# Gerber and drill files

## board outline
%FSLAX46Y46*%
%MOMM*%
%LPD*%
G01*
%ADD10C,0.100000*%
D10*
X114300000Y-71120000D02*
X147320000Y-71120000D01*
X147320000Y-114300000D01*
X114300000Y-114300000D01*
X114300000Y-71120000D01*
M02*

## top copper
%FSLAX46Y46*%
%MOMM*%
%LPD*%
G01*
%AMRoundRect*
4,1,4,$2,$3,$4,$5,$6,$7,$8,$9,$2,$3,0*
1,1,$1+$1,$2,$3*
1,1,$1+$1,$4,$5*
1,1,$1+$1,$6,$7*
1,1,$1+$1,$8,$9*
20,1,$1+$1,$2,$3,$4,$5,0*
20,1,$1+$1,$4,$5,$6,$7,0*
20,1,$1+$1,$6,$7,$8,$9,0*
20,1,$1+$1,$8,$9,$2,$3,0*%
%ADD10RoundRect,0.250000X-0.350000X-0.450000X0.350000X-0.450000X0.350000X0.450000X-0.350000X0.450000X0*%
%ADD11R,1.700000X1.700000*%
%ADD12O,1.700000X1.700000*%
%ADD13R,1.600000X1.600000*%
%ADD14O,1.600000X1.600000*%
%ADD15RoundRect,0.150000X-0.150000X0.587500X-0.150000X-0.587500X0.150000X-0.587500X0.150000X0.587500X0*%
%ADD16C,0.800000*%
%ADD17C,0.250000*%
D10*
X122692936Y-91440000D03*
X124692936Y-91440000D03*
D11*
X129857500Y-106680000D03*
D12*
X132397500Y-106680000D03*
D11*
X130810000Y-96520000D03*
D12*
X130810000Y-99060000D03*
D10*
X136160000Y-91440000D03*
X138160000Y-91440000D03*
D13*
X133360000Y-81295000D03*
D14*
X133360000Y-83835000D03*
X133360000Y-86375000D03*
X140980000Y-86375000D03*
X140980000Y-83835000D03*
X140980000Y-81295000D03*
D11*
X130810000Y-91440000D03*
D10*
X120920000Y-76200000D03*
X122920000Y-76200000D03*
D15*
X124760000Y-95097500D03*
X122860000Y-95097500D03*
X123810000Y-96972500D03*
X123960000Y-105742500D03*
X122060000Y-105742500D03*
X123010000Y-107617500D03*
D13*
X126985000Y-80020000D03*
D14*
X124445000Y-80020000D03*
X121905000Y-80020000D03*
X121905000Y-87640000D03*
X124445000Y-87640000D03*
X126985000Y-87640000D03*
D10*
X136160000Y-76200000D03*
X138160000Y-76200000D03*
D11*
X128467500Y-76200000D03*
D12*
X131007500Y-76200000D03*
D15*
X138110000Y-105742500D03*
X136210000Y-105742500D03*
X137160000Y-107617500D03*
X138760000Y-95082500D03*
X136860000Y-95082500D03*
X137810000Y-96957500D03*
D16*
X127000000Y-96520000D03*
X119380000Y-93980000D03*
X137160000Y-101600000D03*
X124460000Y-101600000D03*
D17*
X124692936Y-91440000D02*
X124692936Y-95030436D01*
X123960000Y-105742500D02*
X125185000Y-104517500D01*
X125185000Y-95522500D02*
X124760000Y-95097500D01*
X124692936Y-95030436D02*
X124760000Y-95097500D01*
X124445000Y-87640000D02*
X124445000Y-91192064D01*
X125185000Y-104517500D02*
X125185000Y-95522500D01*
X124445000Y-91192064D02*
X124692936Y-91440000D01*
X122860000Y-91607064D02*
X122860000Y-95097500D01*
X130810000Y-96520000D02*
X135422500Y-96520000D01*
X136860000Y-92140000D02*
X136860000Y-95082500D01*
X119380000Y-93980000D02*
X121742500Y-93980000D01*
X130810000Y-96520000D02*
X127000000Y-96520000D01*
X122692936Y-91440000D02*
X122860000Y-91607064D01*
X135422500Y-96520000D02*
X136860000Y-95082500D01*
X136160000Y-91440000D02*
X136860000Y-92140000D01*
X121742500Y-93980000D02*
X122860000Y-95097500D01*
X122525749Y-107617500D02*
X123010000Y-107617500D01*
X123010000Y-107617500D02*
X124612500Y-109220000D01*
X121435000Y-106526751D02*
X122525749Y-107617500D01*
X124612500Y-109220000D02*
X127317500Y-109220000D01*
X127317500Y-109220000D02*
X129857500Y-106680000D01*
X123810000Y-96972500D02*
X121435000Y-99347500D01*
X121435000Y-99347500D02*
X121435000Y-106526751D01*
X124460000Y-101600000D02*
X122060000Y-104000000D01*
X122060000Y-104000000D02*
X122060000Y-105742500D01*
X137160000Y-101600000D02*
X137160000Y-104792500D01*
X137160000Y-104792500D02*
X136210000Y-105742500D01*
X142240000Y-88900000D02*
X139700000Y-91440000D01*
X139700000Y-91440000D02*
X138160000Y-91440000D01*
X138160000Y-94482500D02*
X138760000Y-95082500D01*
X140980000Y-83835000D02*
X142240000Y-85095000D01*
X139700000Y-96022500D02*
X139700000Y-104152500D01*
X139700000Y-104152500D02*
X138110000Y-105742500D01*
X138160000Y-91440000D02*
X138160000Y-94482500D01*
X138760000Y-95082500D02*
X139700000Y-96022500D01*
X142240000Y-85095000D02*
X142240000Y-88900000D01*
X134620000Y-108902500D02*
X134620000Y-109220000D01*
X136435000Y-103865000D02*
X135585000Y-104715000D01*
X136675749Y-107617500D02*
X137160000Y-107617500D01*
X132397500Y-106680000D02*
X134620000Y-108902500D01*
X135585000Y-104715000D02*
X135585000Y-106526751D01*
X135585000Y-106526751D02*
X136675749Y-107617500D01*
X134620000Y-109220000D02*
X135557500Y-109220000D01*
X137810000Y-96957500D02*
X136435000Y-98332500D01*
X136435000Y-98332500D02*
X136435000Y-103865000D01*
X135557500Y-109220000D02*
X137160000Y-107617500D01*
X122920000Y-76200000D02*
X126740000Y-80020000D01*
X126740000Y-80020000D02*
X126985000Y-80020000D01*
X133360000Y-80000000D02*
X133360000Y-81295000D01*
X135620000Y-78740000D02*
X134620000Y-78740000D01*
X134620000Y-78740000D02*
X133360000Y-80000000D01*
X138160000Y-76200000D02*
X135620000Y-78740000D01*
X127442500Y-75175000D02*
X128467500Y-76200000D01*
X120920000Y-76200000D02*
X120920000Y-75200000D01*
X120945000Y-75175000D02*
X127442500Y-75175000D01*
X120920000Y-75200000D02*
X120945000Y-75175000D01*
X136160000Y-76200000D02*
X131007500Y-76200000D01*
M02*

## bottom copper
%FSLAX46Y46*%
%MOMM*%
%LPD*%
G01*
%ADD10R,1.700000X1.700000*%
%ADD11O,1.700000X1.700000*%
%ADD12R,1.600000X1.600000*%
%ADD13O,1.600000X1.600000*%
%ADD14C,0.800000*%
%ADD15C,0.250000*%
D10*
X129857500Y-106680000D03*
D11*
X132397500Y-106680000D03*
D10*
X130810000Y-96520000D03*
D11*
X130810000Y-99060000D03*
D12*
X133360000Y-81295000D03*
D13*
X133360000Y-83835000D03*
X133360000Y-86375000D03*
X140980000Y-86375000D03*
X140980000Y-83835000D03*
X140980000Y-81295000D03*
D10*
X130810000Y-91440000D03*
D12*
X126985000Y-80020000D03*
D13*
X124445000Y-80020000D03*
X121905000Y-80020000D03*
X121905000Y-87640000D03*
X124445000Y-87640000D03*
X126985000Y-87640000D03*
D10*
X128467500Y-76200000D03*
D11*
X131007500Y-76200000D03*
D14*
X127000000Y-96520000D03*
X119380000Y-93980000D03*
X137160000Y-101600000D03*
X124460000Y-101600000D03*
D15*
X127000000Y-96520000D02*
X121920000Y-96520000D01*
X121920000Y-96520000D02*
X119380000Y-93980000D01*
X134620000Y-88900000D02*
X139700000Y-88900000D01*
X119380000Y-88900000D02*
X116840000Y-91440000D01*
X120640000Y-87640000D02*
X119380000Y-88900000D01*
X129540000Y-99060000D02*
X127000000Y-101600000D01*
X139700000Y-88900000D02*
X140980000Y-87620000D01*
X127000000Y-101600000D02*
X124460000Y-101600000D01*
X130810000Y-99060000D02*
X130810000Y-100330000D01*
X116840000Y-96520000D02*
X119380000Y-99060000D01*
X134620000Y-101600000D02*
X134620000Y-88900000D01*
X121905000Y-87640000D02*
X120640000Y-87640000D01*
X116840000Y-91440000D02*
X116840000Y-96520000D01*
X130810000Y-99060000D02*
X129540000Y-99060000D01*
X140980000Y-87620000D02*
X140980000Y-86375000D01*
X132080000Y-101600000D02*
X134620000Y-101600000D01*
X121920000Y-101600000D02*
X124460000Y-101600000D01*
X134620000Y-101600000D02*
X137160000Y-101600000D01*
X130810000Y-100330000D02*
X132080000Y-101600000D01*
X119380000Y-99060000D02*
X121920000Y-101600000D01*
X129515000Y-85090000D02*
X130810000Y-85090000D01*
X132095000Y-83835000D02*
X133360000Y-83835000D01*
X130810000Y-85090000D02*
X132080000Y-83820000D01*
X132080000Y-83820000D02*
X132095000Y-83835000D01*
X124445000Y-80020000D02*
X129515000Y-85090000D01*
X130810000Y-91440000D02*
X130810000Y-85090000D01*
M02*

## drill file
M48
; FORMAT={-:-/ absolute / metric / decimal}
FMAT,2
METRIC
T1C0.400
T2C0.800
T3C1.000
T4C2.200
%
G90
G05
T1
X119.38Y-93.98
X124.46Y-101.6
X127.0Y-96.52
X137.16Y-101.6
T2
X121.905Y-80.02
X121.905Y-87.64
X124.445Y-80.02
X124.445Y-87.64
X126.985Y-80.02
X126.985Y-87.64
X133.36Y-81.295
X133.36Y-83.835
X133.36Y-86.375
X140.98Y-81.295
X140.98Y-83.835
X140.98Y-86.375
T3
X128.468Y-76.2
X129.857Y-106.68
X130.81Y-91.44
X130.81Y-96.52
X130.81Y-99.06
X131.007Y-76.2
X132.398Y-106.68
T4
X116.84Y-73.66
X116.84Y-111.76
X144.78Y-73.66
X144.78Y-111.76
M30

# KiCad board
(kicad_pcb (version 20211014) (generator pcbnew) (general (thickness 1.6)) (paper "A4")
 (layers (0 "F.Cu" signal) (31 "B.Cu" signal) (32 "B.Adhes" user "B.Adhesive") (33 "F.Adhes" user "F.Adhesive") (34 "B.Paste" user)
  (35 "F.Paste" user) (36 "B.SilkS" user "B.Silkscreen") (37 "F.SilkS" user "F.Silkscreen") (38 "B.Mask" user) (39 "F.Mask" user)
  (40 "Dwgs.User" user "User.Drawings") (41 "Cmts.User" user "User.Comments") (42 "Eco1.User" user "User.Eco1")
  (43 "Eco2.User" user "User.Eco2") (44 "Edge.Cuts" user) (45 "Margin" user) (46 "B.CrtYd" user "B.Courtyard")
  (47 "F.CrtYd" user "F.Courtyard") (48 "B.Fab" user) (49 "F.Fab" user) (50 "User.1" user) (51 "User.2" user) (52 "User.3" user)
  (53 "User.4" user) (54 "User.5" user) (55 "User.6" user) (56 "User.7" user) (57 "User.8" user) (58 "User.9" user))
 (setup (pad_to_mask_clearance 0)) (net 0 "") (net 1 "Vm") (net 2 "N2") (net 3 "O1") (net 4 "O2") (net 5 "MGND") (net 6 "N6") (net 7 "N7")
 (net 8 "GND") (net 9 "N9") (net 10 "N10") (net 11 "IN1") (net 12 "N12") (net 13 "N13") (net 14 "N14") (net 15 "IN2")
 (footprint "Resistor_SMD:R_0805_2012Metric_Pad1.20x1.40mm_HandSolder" (layer "F.Cu") (at 123.692936 91.44)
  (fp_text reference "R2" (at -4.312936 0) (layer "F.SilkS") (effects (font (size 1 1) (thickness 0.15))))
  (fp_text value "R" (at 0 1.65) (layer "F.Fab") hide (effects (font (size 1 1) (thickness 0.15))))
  (pad "1" smd roundrect (at -1 0) (size 1.2 1.4) (layers "F.Cu" "F.Paste" "F.Mask") (roundrect_rratio 0.208333) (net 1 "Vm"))
  (pad "2" smd roundrect (at 1 0) (size 1.2 1.4) (layers "F.Cu" "F.Paste" "F.Mask") (roundrect_rratio 0.208333) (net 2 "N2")))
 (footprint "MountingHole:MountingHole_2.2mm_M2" (layer "F.Cu") (at 116.84 73.66)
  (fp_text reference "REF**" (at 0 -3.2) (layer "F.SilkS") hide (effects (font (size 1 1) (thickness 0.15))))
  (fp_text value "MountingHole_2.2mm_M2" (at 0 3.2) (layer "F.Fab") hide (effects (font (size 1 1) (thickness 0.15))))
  (pad "" np_thru_hole circle (at 0 0) (size 2.2 2.2) (drill 2.2) (layers *.Cu *.Mask)))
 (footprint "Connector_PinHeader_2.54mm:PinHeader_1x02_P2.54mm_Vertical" (layer "F.Cu") (at 129.8575 106.68 90)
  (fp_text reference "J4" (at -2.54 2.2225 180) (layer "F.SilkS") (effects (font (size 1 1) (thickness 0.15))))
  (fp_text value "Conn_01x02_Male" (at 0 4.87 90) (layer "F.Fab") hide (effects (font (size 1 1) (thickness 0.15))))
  (pad "1" thru_hole rect (at 0 0 90) (size 1.7 1.7) (drill 1) (layers *.Cu *.Mask) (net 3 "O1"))
  (pad "2" thru_hole oval (at 0 2.54 90) (size 1.7 1.7) (drill 1) (layers *.Cu *.Mask) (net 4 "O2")))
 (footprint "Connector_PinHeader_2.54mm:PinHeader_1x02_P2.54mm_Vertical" (layer "F.Cu") (at 130.81 96.52)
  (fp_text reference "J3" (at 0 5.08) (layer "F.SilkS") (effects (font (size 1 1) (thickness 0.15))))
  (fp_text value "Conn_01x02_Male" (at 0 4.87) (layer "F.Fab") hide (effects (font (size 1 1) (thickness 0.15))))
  (pad "1" thru_hole rect (at 0 0) (size 1.7 1.7) (drill 1) (layers *.Cu *.Mask) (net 1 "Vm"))
  (pad "2" thru_hole oval (at 0 2.54) (size 1.7 1.7) (drill 1) (layers *.Cu *.Mask) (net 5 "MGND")))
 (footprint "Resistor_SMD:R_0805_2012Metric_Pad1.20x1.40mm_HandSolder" (layer "F.Cu") (at 137.16 91.44)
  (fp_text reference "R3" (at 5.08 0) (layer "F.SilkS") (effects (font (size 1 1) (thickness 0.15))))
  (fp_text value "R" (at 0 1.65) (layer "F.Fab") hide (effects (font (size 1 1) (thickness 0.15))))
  (pad "1" smd roundrect (at -1 0) (size 1.2 1.4) (layers "F.Cu" "F.Paste" "F.Mask") (roundrect_rratio 0.208333) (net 1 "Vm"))
  (pad "2" smd roundrect (at 1 0) (size 1.2 1.4) (layers "F.Cu" "F.Paste" "F.Mask") (roundrect_rratio 0.208333) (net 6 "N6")))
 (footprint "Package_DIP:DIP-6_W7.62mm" (layer "F.Cu") (at 133.36 81.295)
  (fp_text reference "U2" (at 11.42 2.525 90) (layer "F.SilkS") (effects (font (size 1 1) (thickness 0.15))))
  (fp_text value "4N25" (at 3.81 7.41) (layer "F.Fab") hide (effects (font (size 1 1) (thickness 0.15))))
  (pad "1" thru_hole rect (at 0 0) (size 1.6 1.6) (drill 0.8) (layers *.Cu *.Mask) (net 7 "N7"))
  (pad "2" thru_hole oval (at 0 2.54) (size 1.6 1.6) (drill 0.8) (layers *.Cu *.Mask) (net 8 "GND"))
  (pad "3" thru_hole oval (at 0 5.08) (size 1.6 1.6) (drill 0.8) (layers *.Cu *.Mask) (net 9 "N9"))
  (pad "4" thru_hole oval (at 7.62 5.08) (size 1.6 1.6) (drill 0.8) (layers *.Cu *.Mask) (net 5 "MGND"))
  (pad "5" thru_hole oval (at 7.62 2.54) (size 1.6 1.6) (drill 0.8) (layers *.Cu *.Mask) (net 6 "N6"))
  (pad "6" thru_hole oval (at 7.62 0) (size 1.6 1.6) (drill 0.8) (layers *.Cu *.Mask) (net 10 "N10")))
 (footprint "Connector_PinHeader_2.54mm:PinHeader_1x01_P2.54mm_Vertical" (layer "F.Cu") (at 130.81 91.44)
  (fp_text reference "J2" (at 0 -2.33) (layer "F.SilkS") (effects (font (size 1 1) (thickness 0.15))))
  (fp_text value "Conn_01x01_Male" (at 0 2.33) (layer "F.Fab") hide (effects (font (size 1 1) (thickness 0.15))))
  (pad "1" thru_hole rect (at 0 0) (size 1.7 1.7) (drill 1) (layers *.Cu *.Mask) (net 8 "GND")))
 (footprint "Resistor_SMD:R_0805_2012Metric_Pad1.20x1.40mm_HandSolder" (layer "F.Cu") (at 121.92 76.2)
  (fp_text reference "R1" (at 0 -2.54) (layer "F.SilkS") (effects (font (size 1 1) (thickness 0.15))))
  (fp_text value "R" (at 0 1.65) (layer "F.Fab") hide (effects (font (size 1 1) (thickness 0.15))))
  (pad "1" smd roundrect (at -1 0) (size 1.2 1.4) (layers "F.Cu" "F.Paste" "F.Mask") (roundrect_rratio 0.208333) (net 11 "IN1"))
  (pad "2" smd roundrect (at 1 0) (size 1.2 1.4) (layers "F.Cu" "F.Paste" "F.Mask") (roundrect_rratio 0.208333) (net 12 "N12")))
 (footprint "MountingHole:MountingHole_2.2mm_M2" (layer "F.Cu") (at 144.78 111.76)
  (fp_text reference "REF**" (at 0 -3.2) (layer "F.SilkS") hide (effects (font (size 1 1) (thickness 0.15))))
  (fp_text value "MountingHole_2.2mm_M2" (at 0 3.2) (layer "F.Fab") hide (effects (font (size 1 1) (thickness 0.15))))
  (pad "" np_thru_hole circle (at 0 0) (size 2.2 2.2) (drill 2.2) (layers F&B.Cu *.Mask)))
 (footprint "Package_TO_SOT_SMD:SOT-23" (layer "F.Cu") (at 123.81 96.035 -90)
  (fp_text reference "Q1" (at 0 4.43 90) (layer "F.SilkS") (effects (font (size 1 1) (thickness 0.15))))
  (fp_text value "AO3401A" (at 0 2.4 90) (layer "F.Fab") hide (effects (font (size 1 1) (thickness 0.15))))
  (pad "1" smd roundrect (at -0.9375 -0.95 270) (size 1.475 0.6) (layers "F.Cu" "F.Paste" "F.Mask") (roundrect_rratio 0.25) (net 2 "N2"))
  (pad "2" smd roundrect (at -0.9375 0.95 270) (size 1.475 0.6) (layers "F.Cu" "F.Paste" "F.Mask") (roundrect_rratio 0.25) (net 1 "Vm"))
  (pad "3" smd roundrect (at 0.9375 0 270) (size 1.475 0.6) (layers "F.Cu" "F.Paste" "F.Mask") (roundrect_rratio 0.25) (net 3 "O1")))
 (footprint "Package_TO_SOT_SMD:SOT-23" (layer "F.Cu") (at 123.01 106.68 -90)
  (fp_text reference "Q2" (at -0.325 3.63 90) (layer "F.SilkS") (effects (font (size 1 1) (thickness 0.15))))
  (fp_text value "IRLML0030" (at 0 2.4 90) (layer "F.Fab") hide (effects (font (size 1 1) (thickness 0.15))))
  (pad "1" smd roundrect (at -0.9375 -0.95 270) (size 1.475 0.6) (layers "F.Cu" "F.Paste" "F.Mask") (roundrect_rratio 0.25) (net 2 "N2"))
  (pad "2" smd roundrect (at -0.9375 0.95 270) (size 1.475 0.6) (layers "F.Cu" "F.Paste" "F.Mask") (roundrect_rratio 0.25) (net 5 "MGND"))
  (pad "3" smd roundrect (at 0.9375 0 270) (size 1.475 0.6) (layers "F.Cu" "F.Paste" "F.Mask") (roundrect_rratio 0.25) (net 3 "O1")))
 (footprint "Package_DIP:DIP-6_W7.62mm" (layer "F.Cu") (at 126.985 80.02 -90)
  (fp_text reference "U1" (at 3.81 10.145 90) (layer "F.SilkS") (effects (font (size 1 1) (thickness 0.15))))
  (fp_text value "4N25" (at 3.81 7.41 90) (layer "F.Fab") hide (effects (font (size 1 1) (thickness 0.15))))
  (pad "1" thru_hole rect (at 0 0 270) (size 1.6 1.6) (drill 0.8) (layers *.Cu *.Mask) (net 12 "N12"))
  (pad "2" thru_hole oval (at 0 2.54 270) (size 1.6 1.6) (drill 0.8) (layers *.Cu *.Mask) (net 8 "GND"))
  (pad "3" thru_hole oval (at 0 5.08 270) (size 1.6 1.6) (drill 0.8) (layers *.Cu *.Mask) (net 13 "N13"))
  (pad "4" thru_hole oval (at 7.62 5.08 270) (size 1.6 1.6) (drill 0.8) (layers *.Cu *.Mask) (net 5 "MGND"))
  (pad "5" thru_hole oval (at 7.62 2.54 270) (size 1.6 1.6) (drill 0.8) (layers *.Cu *.Mask) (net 2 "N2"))
  (pad "6" thru_hole oval (at 7.62 0 270) (size 1.6 1.6) (drill 0.8) (layers *.Cu *.Mask) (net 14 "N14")))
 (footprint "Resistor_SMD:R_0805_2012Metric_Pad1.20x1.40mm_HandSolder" (layer "F.Cu") (at 137.16 76.2)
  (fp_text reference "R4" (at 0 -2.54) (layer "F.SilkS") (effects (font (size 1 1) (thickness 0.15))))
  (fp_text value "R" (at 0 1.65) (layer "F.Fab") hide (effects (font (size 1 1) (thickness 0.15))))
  (pad "1" smd roundrect (at -1 0) (size 1.2 1.4) (layers "F.Cu" "F.Paste" "F.Mask") (roundrect_rratio 0.208333) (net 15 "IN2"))
  (pad "2" smd roundrect (at 1 0) (size 1.2 1.4) (layers "F.Cu" "F.Paste" "F.Mask") (roundrect_rratio 0.208333) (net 7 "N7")))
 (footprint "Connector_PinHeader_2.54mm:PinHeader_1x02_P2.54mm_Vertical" (layer "F.Cu") (at 128.4675 76.2 90)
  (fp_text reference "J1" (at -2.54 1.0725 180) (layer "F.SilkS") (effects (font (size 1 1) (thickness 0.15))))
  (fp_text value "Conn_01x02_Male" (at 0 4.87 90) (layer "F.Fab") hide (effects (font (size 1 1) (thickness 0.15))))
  (pad "1" thru_hole rect (at 0 0 90) (size 1.7 1.7) (drill 1) (layers *.Cu *.Mask) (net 11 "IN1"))
  (pad "2" thru_hole oval (at 0 2.54 90) (size 1.7 1.7) (drill 1) (layers *.Cu *.Mask) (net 15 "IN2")))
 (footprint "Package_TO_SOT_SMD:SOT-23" (layer "F.Cu") (at 137.16 106.68 -90)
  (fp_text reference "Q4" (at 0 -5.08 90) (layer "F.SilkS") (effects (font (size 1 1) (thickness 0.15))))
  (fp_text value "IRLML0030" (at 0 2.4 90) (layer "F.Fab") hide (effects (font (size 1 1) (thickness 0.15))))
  (pad "1" smd roundrect (at -0.9375 -0.95 270) (size 1.475 0.6) (layers "F.Cu" "F.Paste" "F.Mask") (roundrect_rratio 0.25) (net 6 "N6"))
  (pad "2" smd roundrect (at -0.9375 0.95 270) (size 1.475 0.6) (layers "F.Cu" "F.Paste" "F.Mask") (roundrect_rratio 0.25) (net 5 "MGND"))
  (pad "3" smd roundrect (at 0.9375 0 270) (size 1.475 0.6) (layers "F.Cu" "F.Paste" "F.Mask") (roundrect_rratio 0.25) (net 4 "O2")))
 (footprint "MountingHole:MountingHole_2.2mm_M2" (layer "F.Cu") (at 116.84 111.76)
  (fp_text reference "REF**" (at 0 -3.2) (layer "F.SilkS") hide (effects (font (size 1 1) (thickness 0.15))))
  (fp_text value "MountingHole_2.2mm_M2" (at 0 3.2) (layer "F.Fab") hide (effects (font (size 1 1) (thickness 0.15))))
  (pad "" np_thru_hole circle (at 0 0) (size 2.2 2.2) (drill 2.2) (layers F&B.Cu *.Mask)))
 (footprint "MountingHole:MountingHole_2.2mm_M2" (layer "F.Cu") (at 144.78 73.66)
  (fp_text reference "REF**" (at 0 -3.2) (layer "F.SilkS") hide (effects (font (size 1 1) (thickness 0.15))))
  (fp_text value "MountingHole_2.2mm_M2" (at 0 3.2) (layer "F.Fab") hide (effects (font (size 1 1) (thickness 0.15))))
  (pad "" np_thru_hole circle (at 0 0) (size 2.2 2.2) (drill 2.2) (layers F&B.Cu *.Mask)))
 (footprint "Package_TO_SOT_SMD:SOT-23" (layer "F.Cu") (at 137.81 96.02 -90)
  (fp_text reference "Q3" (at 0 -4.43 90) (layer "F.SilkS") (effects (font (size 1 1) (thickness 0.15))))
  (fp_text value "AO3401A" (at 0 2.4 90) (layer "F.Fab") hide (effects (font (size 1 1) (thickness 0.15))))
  (pad "1" smd roundrect (at -0.9375 -0.95 270) (size 1.475 0.6) (layers "F.Cu" "F.Paste" "F.Mask") (roundrect_rratio 0.25) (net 6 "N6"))
  (pad "2" smd roundrect (at -0.9375 0.95 270) (size 1.475 0.6) (layers "F.Cu" "F.Paste" "F.Mask") (roundrect_rratio 0.25) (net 1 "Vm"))
  (pad "3" smd roundrect (at 0.9375 0 270) (size 1.475 0.6) (layers "F.Cu" "F.Paste" "F.Mask") (roundrect_rratio 0.25) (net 4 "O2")))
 (gr_rect (start 114.3 71.12) (end 147.32 114.3) (layer "Edge.Cuts") (width 0.1) (fill none))
 (segment (start 124.692936 91.44) (end 124.692936 95.030436) (width 0.25) (layer "F.Cu") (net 2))
 (segment (start 123.96 105.7425) (end 125.185 104.5175) (width 0.25) (layer "F.Cu") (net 2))
 (segment (start 125.185 95.5225) (end 124.76 95.0975) (width 0.25) (layer "F.Cu") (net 2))
 (segment (start 124.692936 95.030436) (end 124.76 95.0975) (width 0.25) (layer "F.Cu") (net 2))
 (segment (start 124.445 87.64) (end 124.445 91.192064) (width 0.25) (layer "F.Cu") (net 2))
 (segment (start 125.185 104.5175) (end 125.185 95.5225) (width 0.25) (layer "F.Cu") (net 2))
 (segment (start 124.445 91.192064) (end 124.692936 91.44) (width 0.25) (layer "F.Cu") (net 2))
 (segment (start 122.86 91.607064) (end 122.86 95.0975) (width 0.25) (layer "F.Cu") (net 1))
 (segment (start 130.81 96.52) (end 135.4225 96.52) (width 0.25) (layer "F.Cu") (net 1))
 (segment (start 136.86 92.14) (end 136.86 95.0825) (width 0.25) (layer "F.Cu") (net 1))
 (segment (start 119.38 93.98) (end 121.7425 93.98) (width 0.25) (layer "F.Cu") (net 1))
 (segment (start 130.81 96.52) (end 127 96.52) (width 0.25) (layer "F.Cu") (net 1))
 (segment (start 122.692936 91.44) (end 122.86 91.607064) (width 0.25) (layer "F.Cu") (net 1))
 (segment (start 135.4225 96.52) (end 136.86 95.0825) (width 0.25) (layer "F.Cu") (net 1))
 (segment (start 136.16 91.44) (end 136.86 92.14) (width 0.25) (layer "F.Cu") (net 1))
 (segment (start 121.7425 93.98) (end 122.86 95.0975) (width 0.25) (layer "F.Cu") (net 1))
 (via (at 127 96.52) (size 0.8) (drill 0.4) (layers "F.Cu" "B.Cu") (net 1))
 (via (at 119.38 93.98) (size 0.8) (drill 0.4) (layers "F.Cu" "B.Cu") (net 1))
 (segment (start 127 96.52) (end 121.92 96.52) (width 0.25) (layer "B.Cu") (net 1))
 (segment (start 121.92 96.52) (end 119.38 93.98) (width 0.25) (layer "B.Cu") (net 1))
 (segment (start 122.525749 107.6175) (end 123.01 107.6175) (width 0.25) (layer "F.Cu") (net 3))
 (segment (start 123.01 107.6175) (end 124.6125 109.22) (width 0.25) (layer "F.Cu") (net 3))
 (segment (start 121.435 106.526751) (end 122.525749 107.6175) (width 0.25) (layer "F.Cu") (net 3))
 (segment (start 124.6125 109.22) (end 127.3175 109.22) (width 0.25) (layer "F.Cu") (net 3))
 (segment (start 127.3175 109.22) (end 129.8575 106.68) (width 0.25) (layer "F.Cu") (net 3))
 (segment (start 123.81 96.9725) (end 121.435 99.3475) (width 0.25) (layer "F.Cu") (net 3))
 (segment (start 121.435 99.3475) (end 121.435 106.526751) (width 0.25) (layer "F.Cu") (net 3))
 (segment (start 124.46 101.6) (end 122.06 104) (width 0.25) (layer "F.Cu") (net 5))
 (segment (start 122.06 104) (end 122.06 105.7425) (width 0.25) (layer "F.Cu") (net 5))
 (segment (start 137.16 101.6) (end 137.16 104.7925) (width 0.25) (layer "F.Cu") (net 5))
 (segment (start 137.16 104.7925) (end 136.21 105.7425) (width 0.25) (layer "F.Cu") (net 5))
 (via (at 137.16 101.6) (size 0.8) (drill 0.4) (layers "F.Cu" "B.Cu") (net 5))
 (via (at 124.46 101.6) (size 0.8) (drill 0.4) (layers "F.Cu" "B.Cu") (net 5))
 (segment (start 134.62 88.9) (end 139.7 88.9) (width 0.25) (layer "B.Cu") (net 5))
 (segment (start 119.38 88.9) (end 116.84 91.44) (width 0.25) (layer "B.Cu") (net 5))
 (segment (start 120.64 87.64) (end 119.38 88.9) (width 0.25) (layer "B.Cu") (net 5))
 (segment (start 129.54 99.06) (end 127 101.6) (width 0.25) (layer "B.Cu") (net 5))
 (segment (start 139.7 88.9) (end 140.98 87.62) (width 0.25) (layer "B.Cu") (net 5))
 (segment (start 127 101.6) (end 124.46 101.6) (width 0.25) (layer "B.Cu") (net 5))
 (segment (start 130.81 99.06) (end 130.81 100.33) (width 0.25) (layer "B.Cu") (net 5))
 (segment (start 116.84 96.52) (end 119.38 99.06) (width 0.25) (layer "B.Cu") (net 5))
 (segment (start 134.62 101.6) (end 134.62 88.9) (width 0.25) (layer "B.Cu") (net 5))
 (segment (start 121.905 87.64) (end 120.64 87.64) (width 0.25) (layer "B.Cu") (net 5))
 (segment (start 116.84 91.44) (end 116.84 96.52) (width 0.25) (layer "B.Cu") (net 5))
 (segment (start 130.81 99.06) (end 129.54 99.06) (width 0.25) (layer "B.Cu") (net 5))
 (segment (start 140.98 87.62) (end 140.98 86.375) (width 0.25) (layer "B.Cu") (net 5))
 (segment (start 132.08 101.6) (end 134.62 101.6) (width 0.25) (layer "B.Cu") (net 5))
 (segment (start 121.92 101.6) (end 124.46 101.6) (width 0.25) (layer "B.Cu") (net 5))
 (segment (start 134.62 101.6) (end 137.16 101.6) (width 0.25) (layer "B.Cu") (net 5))
 (segment (start 130.81 100.33) (end 132.08 101.6) (width 0.25) (layer "B.Cu") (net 5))
 (segment (start 119.38 99.06) (end 121.92 101.6) (width 0.25) (layer "B.Cu") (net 5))
 (segment (start 142.24 88.9) (end 139.7 91.44) (width 0.25) (layer "F.Cu") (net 6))
 (segment (start 139.7 91.44) (end 138.16 91.44) (width 0.25) (layer "F.Cu") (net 6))
 (segment (start 138.16 94.4825) (end 138.76 95.0825) (width 0.25) (layer "F.Cu") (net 6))
 (segment (start 140.98 83.835) (end 142.24 85.095) (width 0.25) (layer "F.Cu") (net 6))
 (segment (start 139.7 96.0225) (end 139.7 104.1525) (width 0.25) (layer "F.Cu") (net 6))
 (segment (start 139.7 104.1525) (end 138.11 105.7425) (width 0.25) (layer "F.Cu") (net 6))
 (segment (start 138.16 91.44) (end 138.16 94.4825) (width 0.25) (layer "F.Cu") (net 6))
 (segment (start 138.76 95.0825) (end 139.7 96.0225) (width 0.25) (layer "F.Cu") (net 6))
 (segment (start 142.24 85.095) (end 142.24 88.9) (width 0.25) (layer "F.Cu") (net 6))
 (segment (start 134.62 108.9025) (end 134.62 109.22) (width 0.25) (layer "F.Cu") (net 4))
 (segment (start 136.435 103.865) (end 135.585 104.715) (width 0.25) (layer "F.Cu") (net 4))
 (segment (start 136.675749 107.6175) (end 137.16 107.6175) (width 0.25) (layer "F.Cu") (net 4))
 (segment (start 132.3975 106.68) (end 134.62 108.9025) (width 0.25) (layer "F.Cu") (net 4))
 (segment (start 135.585 104.715) (end 135.585 106.526751) (width 0.25) (layer "F.Cu") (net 4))
 (segment (start 135.585 106.526751) (end 136.675749 107.6175) (width 0.25) (layer "F.Cu") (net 4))
 (segment (start 134.62 109.22) (end 135.5575 109.22) (width 0.25) (layer "F.Cu") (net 4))
 (segment (start 137.81 96.9575) (end 136.435 98.3325) (width 0.25) (layer "F.Cu") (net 4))
 (segment (start 136.435 98.3325) (end 136.435 103.865) (width 0.25) (layer "F.Cu") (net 4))
 (segment (start 135.5575 109.22) (end 137.16 107.6175) (width 0.25) (layer "F.Cu") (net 4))
 (segment (start 122.92 76.2) (end 126.74 80.02) (width 0.25) (layer "F.Cu") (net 12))
 (segment (start 126.74 80.02) (end 126.985 80.02) (width 0.25) (layer "F.Cu") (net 12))
 (segment (start 129.515 85.09) (end 130.81 85.09) (width 0.25) (layer "B.Cu") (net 8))
 (segment (start 132.095 83.835) (end 133.36 83.835) (width 0.25) (layer "B.Cu") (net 8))
 (segment (start 130.81 85.09) (end 132.08 83.82) (width 0.25) (layer "B.Cu") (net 8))
 (segment (start 132.08 83.82) (end 132.095 83.835) (width 0.25) (layer "B.Cu") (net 8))
 (segment (start 124.445 80.02) (end 129.515 85.09) (width 0.25) (layer "B.Cu") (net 8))
 (segment (start 130.81 91.44) (end 130.81 85.09) (width 0.25) (layer "B.Cu") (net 8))
 (segment (start 133.36 80) (end 133.36 81.295) (width 0.25) (layer "F.Cu") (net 7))
 (segment (start 135.62 78.74) (end 134.62 78.74) (width 0.25) (layer "F.Cu") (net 7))
 (segment (start 134.62 78.74) (end 133.36 80) (width 0.25) (layer "F.Cu") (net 7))
 (segment (start 138.16 76.2) (end 135.62 78.74) (width 0.25) (layer "F.Cu") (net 7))
 (segment (start 127.4425 75.175) (end 128.4675 76.2) (width 0.25) (layer "F.Cu") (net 11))
 (segment (start 120.92 76.2) (end 120.92 75.2) (width 0.25) (layer "F.Cu") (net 11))
 (segment (start 120.945 75.175) (end 127.4425 75.175) (width 0.25) (layer "F.Cu") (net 11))
 (segment (start 120.92 75.2) (end 120.945 75.175) (width 0.25) (layer "F.Cu") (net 11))
 (segment (start 136.16 76.2) (end 131.0075 76.2) (width 0.25) (layer "F.Cu") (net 15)))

